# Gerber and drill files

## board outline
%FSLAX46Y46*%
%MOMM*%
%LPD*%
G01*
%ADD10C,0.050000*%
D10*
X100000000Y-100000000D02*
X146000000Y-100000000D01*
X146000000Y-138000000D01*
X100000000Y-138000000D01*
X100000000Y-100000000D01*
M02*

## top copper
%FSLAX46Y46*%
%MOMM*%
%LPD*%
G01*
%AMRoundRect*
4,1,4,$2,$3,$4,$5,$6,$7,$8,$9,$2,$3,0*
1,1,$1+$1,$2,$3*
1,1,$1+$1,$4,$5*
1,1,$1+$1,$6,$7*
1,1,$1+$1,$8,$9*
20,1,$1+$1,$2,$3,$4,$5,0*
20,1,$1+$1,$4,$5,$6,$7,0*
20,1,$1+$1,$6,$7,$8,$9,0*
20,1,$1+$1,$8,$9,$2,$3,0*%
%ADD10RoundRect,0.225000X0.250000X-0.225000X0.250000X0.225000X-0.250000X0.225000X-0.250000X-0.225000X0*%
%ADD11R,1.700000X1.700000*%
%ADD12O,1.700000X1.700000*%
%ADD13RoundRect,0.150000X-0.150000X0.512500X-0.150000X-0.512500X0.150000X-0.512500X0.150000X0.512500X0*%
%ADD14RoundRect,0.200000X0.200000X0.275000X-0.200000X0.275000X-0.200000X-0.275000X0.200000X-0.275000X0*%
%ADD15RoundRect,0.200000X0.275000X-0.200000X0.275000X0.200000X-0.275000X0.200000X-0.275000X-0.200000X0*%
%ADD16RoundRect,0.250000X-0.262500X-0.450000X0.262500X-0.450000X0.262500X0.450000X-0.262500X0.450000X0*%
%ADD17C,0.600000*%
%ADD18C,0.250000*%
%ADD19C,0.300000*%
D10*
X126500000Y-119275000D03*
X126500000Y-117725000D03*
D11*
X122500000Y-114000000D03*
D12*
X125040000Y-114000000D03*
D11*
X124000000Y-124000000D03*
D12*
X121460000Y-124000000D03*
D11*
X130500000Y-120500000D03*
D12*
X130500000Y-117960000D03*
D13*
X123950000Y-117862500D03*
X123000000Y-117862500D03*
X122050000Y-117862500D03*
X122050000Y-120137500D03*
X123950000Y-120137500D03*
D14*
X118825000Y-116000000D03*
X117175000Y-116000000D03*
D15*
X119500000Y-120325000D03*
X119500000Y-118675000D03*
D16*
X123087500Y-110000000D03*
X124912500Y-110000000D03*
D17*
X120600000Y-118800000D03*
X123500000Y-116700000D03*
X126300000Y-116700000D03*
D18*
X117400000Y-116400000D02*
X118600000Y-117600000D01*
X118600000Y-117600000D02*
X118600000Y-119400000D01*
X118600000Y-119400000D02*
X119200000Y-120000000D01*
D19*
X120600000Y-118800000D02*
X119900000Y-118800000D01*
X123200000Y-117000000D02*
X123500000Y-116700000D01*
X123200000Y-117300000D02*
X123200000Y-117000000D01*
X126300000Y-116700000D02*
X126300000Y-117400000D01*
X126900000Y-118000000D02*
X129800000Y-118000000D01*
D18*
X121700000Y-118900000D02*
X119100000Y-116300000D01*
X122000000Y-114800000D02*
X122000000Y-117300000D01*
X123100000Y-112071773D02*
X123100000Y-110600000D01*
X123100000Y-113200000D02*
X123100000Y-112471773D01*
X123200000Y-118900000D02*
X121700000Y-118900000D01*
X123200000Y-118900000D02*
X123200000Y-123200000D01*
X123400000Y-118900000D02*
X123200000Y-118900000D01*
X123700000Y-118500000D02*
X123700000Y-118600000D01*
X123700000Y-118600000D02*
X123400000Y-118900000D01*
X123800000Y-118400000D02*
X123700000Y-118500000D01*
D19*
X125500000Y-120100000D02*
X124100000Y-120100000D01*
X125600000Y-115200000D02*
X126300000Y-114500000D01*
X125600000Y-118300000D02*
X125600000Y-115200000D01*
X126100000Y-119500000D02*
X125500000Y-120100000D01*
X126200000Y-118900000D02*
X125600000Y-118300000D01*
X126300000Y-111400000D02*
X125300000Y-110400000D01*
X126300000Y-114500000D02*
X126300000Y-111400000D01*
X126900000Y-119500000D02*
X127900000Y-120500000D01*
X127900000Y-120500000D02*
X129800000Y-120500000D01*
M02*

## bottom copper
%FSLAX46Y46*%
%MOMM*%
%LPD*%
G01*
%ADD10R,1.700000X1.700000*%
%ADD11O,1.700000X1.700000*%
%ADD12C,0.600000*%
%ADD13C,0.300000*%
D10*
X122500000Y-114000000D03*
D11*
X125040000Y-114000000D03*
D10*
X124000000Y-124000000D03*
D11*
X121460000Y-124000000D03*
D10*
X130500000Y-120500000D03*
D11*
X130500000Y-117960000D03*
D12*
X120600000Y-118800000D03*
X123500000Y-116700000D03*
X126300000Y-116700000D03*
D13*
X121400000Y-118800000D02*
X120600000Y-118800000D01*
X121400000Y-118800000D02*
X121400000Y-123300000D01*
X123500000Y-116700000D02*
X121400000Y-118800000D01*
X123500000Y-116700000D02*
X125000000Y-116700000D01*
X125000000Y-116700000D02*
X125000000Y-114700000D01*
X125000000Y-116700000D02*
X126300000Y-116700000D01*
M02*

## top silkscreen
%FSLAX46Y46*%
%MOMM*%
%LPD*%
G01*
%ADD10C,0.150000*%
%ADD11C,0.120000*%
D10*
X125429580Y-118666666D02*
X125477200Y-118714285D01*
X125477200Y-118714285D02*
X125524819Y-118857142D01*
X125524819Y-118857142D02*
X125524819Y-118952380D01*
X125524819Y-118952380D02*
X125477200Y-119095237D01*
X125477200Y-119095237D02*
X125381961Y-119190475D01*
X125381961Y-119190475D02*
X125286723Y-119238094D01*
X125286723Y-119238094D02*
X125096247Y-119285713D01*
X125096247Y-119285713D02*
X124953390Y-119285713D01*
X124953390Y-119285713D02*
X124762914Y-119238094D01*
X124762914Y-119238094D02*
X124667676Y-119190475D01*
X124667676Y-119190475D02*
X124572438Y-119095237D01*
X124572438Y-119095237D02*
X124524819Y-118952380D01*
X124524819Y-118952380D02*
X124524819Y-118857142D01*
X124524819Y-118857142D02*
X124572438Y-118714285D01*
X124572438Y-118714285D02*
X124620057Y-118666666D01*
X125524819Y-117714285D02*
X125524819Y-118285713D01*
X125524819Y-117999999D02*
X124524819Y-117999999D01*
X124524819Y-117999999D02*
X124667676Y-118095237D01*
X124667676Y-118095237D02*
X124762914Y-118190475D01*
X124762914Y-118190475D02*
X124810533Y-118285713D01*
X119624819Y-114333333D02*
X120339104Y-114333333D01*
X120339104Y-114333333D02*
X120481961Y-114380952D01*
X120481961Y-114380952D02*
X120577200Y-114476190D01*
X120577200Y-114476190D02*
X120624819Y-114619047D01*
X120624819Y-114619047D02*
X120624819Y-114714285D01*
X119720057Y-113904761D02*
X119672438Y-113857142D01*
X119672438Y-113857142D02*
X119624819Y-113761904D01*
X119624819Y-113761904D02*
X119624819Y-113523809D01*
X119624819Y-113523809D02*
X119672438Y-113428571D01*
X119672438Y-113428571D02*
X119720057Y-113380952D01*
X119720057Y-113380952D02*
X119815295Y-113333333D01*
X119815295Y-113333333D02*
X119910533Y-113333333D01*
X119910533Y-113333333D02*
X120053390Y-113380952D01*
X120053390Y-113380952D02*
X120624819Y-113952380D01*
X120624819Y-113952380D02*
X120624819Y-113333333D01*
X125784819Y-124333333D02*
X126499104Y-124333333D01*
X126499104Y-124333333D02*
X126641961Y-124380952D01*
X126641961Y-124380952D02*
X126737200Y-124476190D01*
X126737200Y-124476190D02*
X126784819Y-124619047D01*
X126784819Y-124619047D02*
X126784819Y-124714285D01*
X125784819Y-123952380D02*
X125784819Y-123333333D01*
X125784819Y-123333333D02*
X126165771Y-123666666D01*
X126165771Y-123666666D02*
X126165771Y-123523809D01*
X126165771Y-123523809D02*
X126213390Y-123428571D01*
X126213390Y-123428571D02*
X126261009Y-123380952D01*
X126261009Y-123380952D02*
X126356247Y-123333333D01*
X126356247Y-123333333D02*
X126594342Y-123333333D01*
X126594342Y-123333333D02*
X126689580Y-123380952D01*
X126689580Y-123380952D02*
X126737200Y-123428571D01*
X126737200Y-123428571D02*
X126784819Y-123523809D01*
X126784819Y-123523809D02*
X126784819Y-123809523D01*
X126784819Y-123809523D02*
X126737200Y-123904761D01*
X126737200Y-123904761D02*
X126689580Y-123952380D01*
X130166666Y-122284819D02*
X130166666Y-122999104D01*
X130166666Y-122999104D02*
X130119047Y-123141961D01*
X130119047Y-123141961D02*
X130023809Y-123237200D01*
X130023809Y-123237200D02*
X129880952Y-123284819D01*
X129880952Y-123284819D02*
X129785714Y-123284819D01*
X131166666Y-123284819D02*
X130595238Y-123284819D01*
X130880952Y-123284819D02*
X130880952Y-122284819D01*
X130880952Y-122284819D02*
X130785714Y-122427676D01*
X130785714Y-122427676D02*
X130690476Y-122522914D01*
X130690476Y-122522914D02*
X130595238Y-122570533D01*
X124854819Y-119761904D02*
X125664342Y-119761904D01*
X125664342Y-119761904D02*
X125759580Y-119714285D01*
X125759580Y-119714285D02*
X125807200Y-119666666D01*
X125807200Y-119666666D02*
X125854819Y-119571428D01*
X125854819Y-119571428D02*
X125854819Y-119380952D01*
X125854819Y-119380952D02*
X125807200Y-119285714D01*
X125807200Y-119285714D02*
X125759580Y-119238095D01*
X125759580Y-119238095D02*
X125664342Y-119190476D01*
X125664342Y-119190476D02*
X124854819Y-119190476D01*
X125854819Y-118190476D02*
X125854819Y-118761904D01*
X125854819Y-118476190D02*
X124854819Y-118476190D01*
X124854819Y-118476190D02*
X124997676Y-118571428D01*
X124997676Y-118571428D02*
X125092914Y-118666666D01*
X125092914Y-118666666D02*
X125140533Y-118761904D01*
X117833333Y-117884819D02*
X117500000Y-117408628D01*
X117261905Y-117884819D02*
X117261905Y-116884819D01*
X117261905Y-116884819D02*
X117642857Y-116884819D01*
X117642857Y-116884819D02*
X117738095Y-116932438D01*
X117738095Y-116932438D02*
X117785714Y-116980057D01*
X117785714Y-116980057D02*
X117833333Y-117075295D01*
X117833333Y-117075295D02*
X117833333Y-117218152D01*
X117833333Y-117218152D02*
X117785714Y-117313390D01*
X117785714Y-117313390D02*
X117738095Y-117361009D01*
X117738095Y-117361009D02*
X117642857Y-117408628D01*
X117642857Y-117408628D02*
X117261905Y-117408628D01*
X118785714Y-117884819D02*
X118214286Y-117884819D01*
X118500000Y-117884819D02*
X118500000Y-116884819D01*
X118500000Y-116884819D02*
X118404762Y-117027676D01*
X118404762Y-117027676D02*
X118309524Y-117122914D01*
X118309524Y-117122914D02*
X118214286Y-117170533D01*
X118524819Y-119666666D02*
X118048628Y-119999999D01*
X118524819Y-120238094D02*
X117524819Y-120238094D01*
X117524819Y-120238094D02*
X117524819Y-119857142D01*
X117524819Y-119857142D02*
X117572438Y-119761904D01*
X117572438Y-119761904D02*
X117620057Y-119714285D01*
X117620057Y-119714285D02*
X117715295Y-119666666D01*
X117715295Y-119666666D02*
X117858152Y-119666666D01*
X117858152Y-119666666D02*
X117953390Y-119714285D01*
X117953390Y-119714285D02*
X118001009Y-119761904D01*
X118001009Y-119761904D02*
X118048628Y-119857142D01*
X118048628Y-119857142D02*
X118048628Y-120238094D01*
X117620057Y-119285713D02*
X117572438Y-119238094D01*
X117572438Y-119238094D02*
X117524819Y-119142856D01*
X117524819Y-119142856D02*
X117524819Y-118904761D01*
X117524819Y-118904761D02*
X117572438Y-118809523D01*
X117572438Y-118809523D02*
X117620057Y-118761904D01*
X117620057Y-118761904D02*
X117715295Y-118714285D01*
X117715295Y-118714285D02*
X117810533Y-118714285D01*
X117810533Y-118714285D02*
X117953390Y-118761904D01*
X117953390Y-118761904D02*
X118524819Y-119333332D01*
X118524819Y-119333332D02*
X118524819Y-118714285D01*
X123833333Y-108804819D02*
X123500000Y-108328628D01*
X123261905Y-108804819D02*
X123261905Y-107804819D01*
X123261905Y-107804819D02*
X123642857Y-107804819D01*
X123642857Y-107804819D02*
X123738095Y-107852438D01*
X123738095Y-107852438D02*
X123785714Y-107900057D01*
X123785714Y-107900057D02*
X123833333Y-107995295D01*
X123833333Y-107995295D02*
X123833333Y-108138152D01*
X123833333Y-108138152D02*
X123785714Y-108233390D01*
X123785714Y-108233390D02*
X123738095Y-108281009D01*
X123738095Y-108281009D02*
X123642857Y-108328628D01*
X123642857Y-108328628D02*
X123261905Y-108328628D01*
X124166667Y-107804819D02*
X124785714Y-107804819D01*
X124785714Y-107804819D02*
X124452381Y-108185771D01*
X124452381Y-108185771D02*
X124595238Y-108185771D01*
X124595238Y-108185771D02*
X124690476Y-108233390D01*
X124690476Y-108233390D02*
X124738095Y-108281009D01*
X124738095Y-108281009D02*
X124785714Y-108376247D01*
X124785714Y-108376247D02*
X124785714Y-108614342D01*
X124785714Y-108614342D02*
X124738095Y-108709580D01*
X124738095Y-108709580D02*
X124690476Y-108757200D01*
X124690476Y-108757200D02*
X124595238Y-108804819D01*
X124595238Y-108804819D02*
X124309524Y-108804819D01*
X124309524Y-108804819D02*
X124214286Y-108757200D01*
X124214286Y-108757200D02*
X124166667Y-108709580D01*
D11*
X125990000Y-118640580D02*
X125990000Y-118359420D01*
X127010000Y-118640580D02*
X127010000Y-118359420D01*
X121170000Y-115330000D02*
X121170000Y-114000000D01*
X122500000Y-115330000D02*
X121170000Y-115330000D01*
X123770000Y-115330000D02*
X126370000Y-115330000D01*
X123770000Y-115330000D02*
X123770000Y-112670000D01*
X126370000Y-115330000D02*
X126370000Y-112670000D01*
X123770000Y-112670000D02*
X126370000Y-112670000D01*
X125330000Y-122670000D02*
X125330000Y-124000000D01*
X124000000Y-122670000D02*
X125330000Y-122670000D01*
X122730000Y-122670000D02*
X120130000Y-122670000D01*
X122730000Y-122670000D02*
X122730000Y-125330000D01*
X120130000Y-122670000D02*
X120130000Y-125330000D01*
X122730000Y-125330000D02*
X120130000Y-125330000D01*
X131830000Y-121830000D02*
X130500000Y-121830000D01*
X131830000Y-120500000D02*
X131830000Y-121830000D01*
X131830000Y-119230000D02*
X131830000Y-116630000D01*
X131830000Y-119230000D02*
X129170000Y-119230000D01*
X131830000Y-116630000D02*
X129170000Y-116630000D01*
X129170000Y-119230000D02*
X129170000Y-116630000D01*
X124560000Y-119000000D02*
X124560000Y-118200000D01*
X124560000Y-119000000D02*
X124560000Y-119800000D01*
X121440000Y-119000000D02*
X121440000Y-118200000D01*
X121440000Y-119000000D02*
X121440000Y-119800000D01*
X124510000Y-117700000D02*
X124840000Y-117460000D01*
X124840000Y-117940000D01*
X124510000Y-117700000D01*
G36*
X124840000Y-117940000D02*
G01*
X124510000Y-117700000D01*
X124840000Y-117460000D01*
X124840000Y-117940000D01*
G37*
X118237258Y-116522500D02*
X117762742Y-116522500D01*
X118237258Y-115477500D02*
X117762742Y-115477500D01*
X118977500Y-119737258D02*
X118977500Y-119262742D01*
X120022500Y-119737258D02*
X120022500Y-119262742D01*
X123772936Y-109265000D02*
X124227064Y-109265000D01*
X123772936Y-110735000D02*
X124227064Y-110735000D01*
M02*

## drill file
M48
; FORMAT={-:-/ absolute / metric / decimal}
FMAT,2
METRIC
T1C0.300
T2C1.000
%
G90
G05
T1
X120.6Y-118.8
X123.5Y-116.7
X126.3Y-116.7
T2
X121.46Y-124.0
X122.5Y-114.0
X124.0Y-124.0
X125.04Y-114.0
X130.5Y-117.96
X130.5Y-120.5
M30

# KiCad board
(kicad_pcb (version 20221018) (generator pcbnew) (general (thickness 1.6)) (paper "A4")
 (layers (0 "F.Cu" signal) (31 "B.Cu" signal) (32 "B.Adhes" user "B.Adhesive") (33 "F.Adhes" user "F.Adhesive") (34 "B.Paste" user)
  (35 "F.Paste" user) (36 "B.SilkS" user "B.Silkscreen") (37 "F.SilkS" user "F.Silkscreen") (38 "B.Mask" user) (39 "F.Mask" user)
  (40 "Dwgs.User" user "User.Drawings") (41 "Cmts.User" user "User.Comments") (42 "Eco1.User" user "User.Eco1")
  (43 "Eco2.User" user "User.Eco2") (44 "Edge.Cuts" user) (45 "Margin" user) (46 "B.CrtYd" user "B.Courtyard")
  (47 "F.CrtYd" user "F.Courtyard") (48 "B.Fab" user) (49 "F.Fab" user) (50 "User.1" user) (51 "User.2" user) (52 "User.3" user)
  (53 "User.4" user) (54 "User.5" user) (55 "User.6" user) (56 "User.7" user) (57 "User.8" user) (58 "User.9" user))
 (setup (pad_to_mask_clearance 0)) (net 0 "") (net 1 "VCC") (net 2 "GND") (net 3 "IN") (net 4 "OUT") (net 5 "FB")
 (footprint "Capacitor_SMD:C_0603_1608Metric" (layer "F.Cu") (at 126.5 118.5 90)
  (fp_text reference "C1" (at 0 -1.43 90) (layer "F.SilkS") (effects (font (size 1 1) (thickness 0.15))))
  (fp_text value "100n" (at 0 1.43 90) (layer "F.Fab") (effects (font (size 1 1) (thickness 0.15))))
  (fp_line (start -0.14058 -0.51) (end 0.14058 -0.51) (stroke (width 0.12) (type solid)) (layer "F.SilkS"))
  (fp_line (start -0.14058 0.51) (end 0.14058 0.51) (stroke (width 0.12) (type solid)) (layer "F.SilkS"))
  (pad "1" smd roundrect (at -0.775 0 90) (size 0.9 0.95) (layers "F.Cu" "F.Paste" "F.Mask") (roundrect_rratio 0.25) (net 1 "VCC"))
  (pad "2" smd roundrect (at 0.775 0 90) (size 0.9 0.95) (layers "F.Cu" "F.Paste" "F.Mask") (roundrect_rratio 0.25) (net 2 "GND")))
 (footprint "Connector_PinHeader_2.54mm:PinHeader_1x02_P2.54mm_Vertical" (layer "F.Cu") (at 122.5 114 90)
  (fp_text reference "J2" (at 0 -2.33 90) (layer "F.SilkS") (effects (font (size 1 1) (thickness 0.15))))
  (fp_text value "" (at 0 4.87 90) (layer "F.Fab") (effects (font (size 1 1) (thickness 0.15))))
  (fp_line (start -1.33 -1.33) (end 0 -1.33) (stroke (width 0.12) (type solid)) (layer "F.SilkS"))
  (fp_line (start -1.33 0) (end -1.33 -1.33) (stroke (width 0.12) (type solid)) (layer "F.SilkS"))
  (fp_line (start -1.33 1.27) (end -1.33 3.87) (stroke (width 0.12) (type solid)) (layer "F.SilkS"))
  (fp_line (start -1.33 1.27) (end 1.33 1.27) (stroke (width 0.12) (type solid)) (layer "F.SilkS"))
  (fp_line (start -1.33 3.87) (end 1.33 3.87) (stroke (width 0.12) (type solid)) (layer "F.SilkS"))
  (fp_line (start 1.33 1.27) (end 1.33 3.87) (stroke (width 0.12) (type solid)) (layer "F.SilkS"))
  (pad "1" thru_hole rect (at 0 0 90) (size 1.7 1.7) (drill 1) (layers "*.Cu" "*.Mask") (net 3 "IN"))
  (pad "2" thru_hole oval (at 0 2.54 90) (size 1.7 1.7) (drill 1) (layers "*.Cu" "*.Mask") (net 2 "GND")))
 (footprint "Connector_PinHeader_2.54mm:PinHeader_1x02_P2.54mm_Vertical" (layer "F.Cu") (at 124 124 -90)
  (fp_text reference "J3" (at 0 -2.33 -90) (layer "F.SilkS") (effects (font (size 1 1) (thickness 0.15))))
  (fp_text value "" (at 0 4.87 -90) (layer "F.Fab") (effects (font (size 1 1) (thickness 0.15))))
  (fp_line (start -1.33 -1.33) (end 0 -1.33) (stroke (width 0.12) (type solid)) (layer "F.SilkS"))
  (fp_line (start -1.33 0) (end -1.33 -1.33) (stroke (width 0.12) (type solid)) (layer "F.SilkS"))
  (fp_line (start -1.33 1.27) (end -1.33 3.87) (stroke (width 0.12) (type solid)) (layer "F.SilkS"))
  (fp_line (start -1.33 1.27) (end 1.33 1.27) (stroke (width 0.12) (type solid)) (layer "F.SilkS"))
  (fp_line (start -1.33 3.87) (end 1.33 3.87) (stroke (width 0.12) (type solid)) (layer "F.SilkS"))
  (fp_line (start 1.33 1.27) (end 1.33 3.87) (stroke (width 0.12) (type solid)) (layer "F.SilkS"))
  (pad "1" thru_hole rect (at 0 0 270) (size 1.7 1.7) (drill 1) (layers "*.Cu" "*.Mask") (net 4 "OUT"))
  (pad "2" thru_hole oval (at 0 2.54 270) (size 1.7 1.7) (drill 1) (layers "*.Cu" "*.Mask") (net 2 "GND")))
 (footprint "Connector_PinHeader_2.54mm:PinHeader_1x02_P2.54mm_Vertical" (layer "F.Cu") (at 130.5 120.5 180)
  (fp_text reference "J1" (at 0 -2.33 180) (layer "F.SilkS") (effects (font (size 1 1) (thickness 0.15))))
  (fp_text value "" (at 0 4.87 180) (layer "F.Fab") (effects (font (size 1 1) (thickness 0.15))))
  (fp_line (start -1.33 -1.33) (end 0 -1.33) (stroke (width 0.12) (type solid)) (layer "F.SilkS"))
  (fp_line (start -1.33 0) (end -1.33 -1.33) (stroke (width 0.12) (type solid)) (layer "F.SilkS"))
  (fp_line (start -1.33 1.27) (end -1.33 3.87) (stroke (width 0.12) (type solid)) (layer "F.SilkS"))
  (fp_line (start -1.33 1.27) (end 1.33 1.27) (stroke (width 0.12) (type solid)) (layer "F.SilkS"))
  (fp_line (start -1.33 3.87) (end 1.33 3.87) (stroke (width 0.12) (type solid)) (layer "F.SilkS"))
  (fp_line (start 1.33 1.27) (end 1.33 3.87) (stroke (width 0.12) (type solid)) (layer "F.SilkS"))
  (pad "1" thru_hole rect (at 0 0 180) (size 1.7 1.7) (drill 1) (layers "*.Cu" "*.Mask") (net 1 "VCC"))
  (pad "2" thru_hole oval (at 0 2.54 180) (size 1.7 1.7) (drill 1) (layers "*.Cu" "*.Mask") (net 2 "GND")))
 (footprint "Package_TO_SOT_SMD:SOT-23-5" (layer "F.Cu") (at 123 119 -90)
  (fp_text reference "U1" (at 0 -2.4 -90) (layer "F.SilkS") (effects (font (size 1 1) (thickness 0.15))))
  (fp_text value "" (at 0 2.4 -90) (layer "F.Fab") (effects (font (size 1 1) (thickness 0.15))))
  (fp_line (start 0 -1.56) (end -0.8 -1.56) (stroke (width 0.12) (type solid)) (layer "F.SilkS"))
  (fp_line (start 0 -1.56) (end 0.8 -1.56) (stroke (width 0.12) (type solid)) (layer "F.SilkS"))
  (fp_line (start 0 1.56) (end -0.8 1.56) (stroke (width 0.12) (type solid)) (layer "F.SilkS"))
  (fp_line (start 0 1.56) (end 0.8 1.56) (stroke (width 0.12) (type solid)) (layer "F.SilkS"))
  (fp_poly
   (pts (xy -1.3 -1.51) (xy -1.54 -1.84) (xy -1.06 -1.84) (xy -1.3 -1.51)) (stroke (width 0.12) (type solid)) (fill solid) (layer "F.SilkS"))
  (pad "1" smd roundrect (at -1.1375 -0.95 270) (size 1.325 0.6) (layers "F.Cu" "F.Paste" "F.Mask") (roundrect_rratio 0.25) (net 4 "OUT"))
  (pad "2" smd roundrect (at -1.1375 0 270) (size 1.325 0.6) (layers "F.Cu" "F.Paste" "F.Mask") (roundrect_rratio 0.25) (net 2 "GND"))
  (pad "3" smd roundrect (at -1.1375 0.95 270) (size 1.325 0.6) (layers "F.Cu" "F.Paste" "F.Mask") (roundrect_rratio 0.25) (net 3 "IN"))
  (pad "4" smd roundrect (at 1.1375 0.95 270) (size 1.325 0.6) (layers "F.Cu" "F.Paste" "F.Mask") (roundrect_rratio 0.25))
  (pad "5" smd roundrect (at 1.1375 -0.95 270) (size 1.325 0.6) (layers "F.Cu" "F.Paste" "F.Mask") (roundrect_rratio 0.25) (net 1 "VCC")))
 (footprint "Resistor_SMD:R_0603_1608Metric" (layer "F.Cu") (at 118 116 180)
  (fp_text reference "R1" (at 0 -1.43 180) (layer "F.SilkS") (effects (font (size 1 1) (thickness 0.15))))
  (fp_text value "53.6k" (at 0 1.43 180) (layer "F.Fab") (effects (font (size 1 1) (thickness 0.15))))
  (fp_line (start -0.237258 -0.5225) (end 0.237258 -0.5225) (stroke (width 0.12) (type solid)) (layer "F.SilkS"))
  (fp_line (start -0.237258 0.5225) (end 0.237258 0.5225) (stroke (width 0.12) (type solid)) (layer "F.SilkS"))
  (pad "1" smd roundrect (at -0.825 0 180) (size 0.8 0.95) (layers "F.Cu" "F.Paste" "F.Mask") (roundrect_rratio 0.25) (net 4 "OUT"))
  (pad "2" smd roundrect (at 0.825 0 180) (size 0.8 0.95) (layers "F.Cu" "F.Paste" "F.Mask") (roundrect_rratio 0.25) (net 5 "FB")))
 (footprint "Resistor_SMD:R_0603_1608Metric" (layer "F.Cu") (at 119.5 119.5 90)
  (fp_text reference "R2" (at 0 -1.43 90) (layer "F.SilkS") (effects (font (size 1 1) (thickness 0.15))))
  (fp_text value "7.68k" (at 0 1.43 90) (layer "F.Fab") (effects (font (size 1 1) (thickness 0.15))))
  (fp_line (start -0.237258 -0.5225) (end 0.237258 -0.5225) (stroke (width 0.12) (type solid)) (layer "F.SilkS"))
  (fp_line (start -0.237258 0.5225) (end 0.237258 0.5225) (stroke (width 0.12) (type solid)) (layer "F.SilkS"))
  (pad "1" smd roundrect (at -0.825 0 90) (size 0.8 0.95) (layers "F.Cu" "F.Paste" "F.Mask") (roundrect_rratio 0.25) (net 5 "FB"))
  (pad "2" smd roundrect (at 0.825 0 90) (size 0.8 0.95) (layers "F.Cu" "F.Paste" "F.Mask") (roundrect_rratio 0.25) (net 2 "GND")))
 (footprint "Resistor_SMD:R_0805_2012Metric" (layer "F.Cu") (at 124 110)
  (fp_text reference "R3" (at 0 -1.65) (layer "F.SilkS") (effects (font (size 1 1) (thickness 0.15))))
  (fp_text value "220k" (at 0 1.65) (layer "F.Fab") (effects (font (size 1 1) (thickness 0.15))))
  (fp_line (start -0.227064 -0.735) (end 0.227064 -0.735) (stroke (width 0.12) (type solid)) (layer "F.SilkS"))
  (fp_line (start -0.227064 0.735) (end 0.227064 0.735) (stroke (width 0.12) (type solid)) (layer "F.SilkS"))
  (pad "1" smd roundrect (at -0.9125 0) (size 1.025 1.4) (layers "F.Cu" "F.Paste" "F.Mask") (roundrect_rratio 0.243902) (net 3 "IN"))
  (pad "2" smd roundrect (at 0.9125 0) (size 1.025 1.4) (layers "F.Cu" "F.Paste" "F.Mask") (roundrect_rratio 0.243902) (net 1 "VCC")))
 (gr_rect (start 100 100) (end 146 138) (stroke (width 0.05) (type default)) (fill none) (layer "Edge.Cuts"))
 (segment (start 117.4 116.4) (end 118.6 117.6) (width 0.25) (layer "F.Cu") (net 5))
 (segment (start 118.6 117.6) (end 118.6 119.4) (width 0.25) (layer "F.Cu") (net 5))
 (segment (start 118.6 119.4) (end 119.2 120) (width 0.25) (layer "F.Cu") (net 5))
 (segment (start 120.6 118.8) (end 119.9 118.8) (width 0.3) (layer "F.Cu") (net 2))
 (segment (start 123.2 117) (end 123.5 116.7) (width 0.3) (layer "F.Cu") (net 2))
 (segment (start 123.2 117.3) (end 123.2 117) (width 0.3) (layer "F.Cu") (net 2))
 (segment (start 126.3 116.7) (end 126.3 117.4) (width 0.3) (layer "F.Cu") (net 2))
 (segment (start 126.9 118) (end 129.8 118) (width 0.3) (layer "F.Cu") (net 2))
 (via (at 120.6 118.8) (size 0.6) (drill 0.3) (layers "F.Cu" "B.Cu") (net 2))
 (via (at 123.5 116.7) (size 0.6) (drill 0.3) (layers "F.Cu" "B.Cu") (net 2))
 (via (at 126.3 116.7) (size 0.6) (drill 0.3) (layers "F.Cu" "B.Cu") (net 2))
 (segment (start 121.4 118.8) (end 120.6 118.8) (width 0.3) (layer "B.Cu") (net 2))
 (segment (start 121.4 118.8) (end 121.4 123.3) (width 0.3) (layer "B.Cu") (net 2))
 (segment (start 121.7 118.9) (end 119.1 116.3) (width 0.25) (layer "F.Cu") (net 4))
 (segment (start 122 114.8) (end 122 117.3) (width 0.25) (layer "F.Cu") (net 3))
 (segment (start 123.1 112.071773) (end 123.1 110.6) (width 0.25) (layer "F.Cu") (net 3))
 (segment (start 123.1 113.2) (end 123.1 112.471773) (width 0.25) (layer "F.Cu") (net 3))
 (segment (start 123.2 118.9) (end 121.7 118.9) (width 0.25) (layer "F.Cu") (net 4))
 (segment (start 123.2 118.9) (end 123.2 123.2) (width 0.25) (layer "F.Cu") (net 4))
 (segment (start 123.4 118.9) (end 123.2 118.9) (width 0.25) (layer "F.Cu") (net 4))
 (segment (start 123.5 116.7) (end 121.4 118.8) (width 0.3) (layer "B.Cu") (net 2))
 (segment (start 123.5 116.7) (end 125 116.7) (width 0.3) (layer "B.Cu") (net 2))
 (segment (start 123.7 118.5) (end 123.7 118.6) (width 0.25) (layer "F.Cu") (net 4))
 (segment (start 123.7 118.6) (end 123.4 118.9) (width 0.25) (layer "F.Cu") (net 4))
 (segment (start 123.8 118.4) (end 123.7 118.5) (width 0.25) (layer "F.Cu") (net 4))
 (segment (start 125 116.7) (end 125 114.7) (width 0.3) (layer "B.Cu") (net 2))
 (segment (start 125 116.7) (end 126.3 116.7) (width 0.3) (layer "B.Cu") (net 2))
 (segment (start 125.5 120.1) (end 124.1 120.1) (width 0.3) (layer "F.Cu") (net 1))
 (segment (start 125.6 115.2) (end 126.3 114.5) (width 0.3) (layer "F.Cu") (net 1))
 (segment (start 125.6 118.3) (end 125.6 115.2) (width 0.3) (layer "F.Cu") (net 1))
 (segment (start 126.1 119.5) (end 125.5 120.1) (width 0.3) (layer "F.Cu") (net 1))
 (segment (start 126.2 118.9) (end 125.6 118.3) (width 0.3) (layer "F.Cu") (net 1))
 (segment (start 126.3 111.4) (end 125.3 110.4) (width 0.3) (layer "F.Cu") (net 1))
 (segment (start 126.3 114.5) (end 126.3 111.4) (width 0.3) (layer "F.Cu") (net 1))
 (segment (start 126.9 119.5) (end 127.9 120.5) (width 0.3) (layer "F.Cu") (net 1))
 (segment (start 127.9 120.5) (end 129.8 120.5) (width 0.3) (layer "F.Cu") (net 1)))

